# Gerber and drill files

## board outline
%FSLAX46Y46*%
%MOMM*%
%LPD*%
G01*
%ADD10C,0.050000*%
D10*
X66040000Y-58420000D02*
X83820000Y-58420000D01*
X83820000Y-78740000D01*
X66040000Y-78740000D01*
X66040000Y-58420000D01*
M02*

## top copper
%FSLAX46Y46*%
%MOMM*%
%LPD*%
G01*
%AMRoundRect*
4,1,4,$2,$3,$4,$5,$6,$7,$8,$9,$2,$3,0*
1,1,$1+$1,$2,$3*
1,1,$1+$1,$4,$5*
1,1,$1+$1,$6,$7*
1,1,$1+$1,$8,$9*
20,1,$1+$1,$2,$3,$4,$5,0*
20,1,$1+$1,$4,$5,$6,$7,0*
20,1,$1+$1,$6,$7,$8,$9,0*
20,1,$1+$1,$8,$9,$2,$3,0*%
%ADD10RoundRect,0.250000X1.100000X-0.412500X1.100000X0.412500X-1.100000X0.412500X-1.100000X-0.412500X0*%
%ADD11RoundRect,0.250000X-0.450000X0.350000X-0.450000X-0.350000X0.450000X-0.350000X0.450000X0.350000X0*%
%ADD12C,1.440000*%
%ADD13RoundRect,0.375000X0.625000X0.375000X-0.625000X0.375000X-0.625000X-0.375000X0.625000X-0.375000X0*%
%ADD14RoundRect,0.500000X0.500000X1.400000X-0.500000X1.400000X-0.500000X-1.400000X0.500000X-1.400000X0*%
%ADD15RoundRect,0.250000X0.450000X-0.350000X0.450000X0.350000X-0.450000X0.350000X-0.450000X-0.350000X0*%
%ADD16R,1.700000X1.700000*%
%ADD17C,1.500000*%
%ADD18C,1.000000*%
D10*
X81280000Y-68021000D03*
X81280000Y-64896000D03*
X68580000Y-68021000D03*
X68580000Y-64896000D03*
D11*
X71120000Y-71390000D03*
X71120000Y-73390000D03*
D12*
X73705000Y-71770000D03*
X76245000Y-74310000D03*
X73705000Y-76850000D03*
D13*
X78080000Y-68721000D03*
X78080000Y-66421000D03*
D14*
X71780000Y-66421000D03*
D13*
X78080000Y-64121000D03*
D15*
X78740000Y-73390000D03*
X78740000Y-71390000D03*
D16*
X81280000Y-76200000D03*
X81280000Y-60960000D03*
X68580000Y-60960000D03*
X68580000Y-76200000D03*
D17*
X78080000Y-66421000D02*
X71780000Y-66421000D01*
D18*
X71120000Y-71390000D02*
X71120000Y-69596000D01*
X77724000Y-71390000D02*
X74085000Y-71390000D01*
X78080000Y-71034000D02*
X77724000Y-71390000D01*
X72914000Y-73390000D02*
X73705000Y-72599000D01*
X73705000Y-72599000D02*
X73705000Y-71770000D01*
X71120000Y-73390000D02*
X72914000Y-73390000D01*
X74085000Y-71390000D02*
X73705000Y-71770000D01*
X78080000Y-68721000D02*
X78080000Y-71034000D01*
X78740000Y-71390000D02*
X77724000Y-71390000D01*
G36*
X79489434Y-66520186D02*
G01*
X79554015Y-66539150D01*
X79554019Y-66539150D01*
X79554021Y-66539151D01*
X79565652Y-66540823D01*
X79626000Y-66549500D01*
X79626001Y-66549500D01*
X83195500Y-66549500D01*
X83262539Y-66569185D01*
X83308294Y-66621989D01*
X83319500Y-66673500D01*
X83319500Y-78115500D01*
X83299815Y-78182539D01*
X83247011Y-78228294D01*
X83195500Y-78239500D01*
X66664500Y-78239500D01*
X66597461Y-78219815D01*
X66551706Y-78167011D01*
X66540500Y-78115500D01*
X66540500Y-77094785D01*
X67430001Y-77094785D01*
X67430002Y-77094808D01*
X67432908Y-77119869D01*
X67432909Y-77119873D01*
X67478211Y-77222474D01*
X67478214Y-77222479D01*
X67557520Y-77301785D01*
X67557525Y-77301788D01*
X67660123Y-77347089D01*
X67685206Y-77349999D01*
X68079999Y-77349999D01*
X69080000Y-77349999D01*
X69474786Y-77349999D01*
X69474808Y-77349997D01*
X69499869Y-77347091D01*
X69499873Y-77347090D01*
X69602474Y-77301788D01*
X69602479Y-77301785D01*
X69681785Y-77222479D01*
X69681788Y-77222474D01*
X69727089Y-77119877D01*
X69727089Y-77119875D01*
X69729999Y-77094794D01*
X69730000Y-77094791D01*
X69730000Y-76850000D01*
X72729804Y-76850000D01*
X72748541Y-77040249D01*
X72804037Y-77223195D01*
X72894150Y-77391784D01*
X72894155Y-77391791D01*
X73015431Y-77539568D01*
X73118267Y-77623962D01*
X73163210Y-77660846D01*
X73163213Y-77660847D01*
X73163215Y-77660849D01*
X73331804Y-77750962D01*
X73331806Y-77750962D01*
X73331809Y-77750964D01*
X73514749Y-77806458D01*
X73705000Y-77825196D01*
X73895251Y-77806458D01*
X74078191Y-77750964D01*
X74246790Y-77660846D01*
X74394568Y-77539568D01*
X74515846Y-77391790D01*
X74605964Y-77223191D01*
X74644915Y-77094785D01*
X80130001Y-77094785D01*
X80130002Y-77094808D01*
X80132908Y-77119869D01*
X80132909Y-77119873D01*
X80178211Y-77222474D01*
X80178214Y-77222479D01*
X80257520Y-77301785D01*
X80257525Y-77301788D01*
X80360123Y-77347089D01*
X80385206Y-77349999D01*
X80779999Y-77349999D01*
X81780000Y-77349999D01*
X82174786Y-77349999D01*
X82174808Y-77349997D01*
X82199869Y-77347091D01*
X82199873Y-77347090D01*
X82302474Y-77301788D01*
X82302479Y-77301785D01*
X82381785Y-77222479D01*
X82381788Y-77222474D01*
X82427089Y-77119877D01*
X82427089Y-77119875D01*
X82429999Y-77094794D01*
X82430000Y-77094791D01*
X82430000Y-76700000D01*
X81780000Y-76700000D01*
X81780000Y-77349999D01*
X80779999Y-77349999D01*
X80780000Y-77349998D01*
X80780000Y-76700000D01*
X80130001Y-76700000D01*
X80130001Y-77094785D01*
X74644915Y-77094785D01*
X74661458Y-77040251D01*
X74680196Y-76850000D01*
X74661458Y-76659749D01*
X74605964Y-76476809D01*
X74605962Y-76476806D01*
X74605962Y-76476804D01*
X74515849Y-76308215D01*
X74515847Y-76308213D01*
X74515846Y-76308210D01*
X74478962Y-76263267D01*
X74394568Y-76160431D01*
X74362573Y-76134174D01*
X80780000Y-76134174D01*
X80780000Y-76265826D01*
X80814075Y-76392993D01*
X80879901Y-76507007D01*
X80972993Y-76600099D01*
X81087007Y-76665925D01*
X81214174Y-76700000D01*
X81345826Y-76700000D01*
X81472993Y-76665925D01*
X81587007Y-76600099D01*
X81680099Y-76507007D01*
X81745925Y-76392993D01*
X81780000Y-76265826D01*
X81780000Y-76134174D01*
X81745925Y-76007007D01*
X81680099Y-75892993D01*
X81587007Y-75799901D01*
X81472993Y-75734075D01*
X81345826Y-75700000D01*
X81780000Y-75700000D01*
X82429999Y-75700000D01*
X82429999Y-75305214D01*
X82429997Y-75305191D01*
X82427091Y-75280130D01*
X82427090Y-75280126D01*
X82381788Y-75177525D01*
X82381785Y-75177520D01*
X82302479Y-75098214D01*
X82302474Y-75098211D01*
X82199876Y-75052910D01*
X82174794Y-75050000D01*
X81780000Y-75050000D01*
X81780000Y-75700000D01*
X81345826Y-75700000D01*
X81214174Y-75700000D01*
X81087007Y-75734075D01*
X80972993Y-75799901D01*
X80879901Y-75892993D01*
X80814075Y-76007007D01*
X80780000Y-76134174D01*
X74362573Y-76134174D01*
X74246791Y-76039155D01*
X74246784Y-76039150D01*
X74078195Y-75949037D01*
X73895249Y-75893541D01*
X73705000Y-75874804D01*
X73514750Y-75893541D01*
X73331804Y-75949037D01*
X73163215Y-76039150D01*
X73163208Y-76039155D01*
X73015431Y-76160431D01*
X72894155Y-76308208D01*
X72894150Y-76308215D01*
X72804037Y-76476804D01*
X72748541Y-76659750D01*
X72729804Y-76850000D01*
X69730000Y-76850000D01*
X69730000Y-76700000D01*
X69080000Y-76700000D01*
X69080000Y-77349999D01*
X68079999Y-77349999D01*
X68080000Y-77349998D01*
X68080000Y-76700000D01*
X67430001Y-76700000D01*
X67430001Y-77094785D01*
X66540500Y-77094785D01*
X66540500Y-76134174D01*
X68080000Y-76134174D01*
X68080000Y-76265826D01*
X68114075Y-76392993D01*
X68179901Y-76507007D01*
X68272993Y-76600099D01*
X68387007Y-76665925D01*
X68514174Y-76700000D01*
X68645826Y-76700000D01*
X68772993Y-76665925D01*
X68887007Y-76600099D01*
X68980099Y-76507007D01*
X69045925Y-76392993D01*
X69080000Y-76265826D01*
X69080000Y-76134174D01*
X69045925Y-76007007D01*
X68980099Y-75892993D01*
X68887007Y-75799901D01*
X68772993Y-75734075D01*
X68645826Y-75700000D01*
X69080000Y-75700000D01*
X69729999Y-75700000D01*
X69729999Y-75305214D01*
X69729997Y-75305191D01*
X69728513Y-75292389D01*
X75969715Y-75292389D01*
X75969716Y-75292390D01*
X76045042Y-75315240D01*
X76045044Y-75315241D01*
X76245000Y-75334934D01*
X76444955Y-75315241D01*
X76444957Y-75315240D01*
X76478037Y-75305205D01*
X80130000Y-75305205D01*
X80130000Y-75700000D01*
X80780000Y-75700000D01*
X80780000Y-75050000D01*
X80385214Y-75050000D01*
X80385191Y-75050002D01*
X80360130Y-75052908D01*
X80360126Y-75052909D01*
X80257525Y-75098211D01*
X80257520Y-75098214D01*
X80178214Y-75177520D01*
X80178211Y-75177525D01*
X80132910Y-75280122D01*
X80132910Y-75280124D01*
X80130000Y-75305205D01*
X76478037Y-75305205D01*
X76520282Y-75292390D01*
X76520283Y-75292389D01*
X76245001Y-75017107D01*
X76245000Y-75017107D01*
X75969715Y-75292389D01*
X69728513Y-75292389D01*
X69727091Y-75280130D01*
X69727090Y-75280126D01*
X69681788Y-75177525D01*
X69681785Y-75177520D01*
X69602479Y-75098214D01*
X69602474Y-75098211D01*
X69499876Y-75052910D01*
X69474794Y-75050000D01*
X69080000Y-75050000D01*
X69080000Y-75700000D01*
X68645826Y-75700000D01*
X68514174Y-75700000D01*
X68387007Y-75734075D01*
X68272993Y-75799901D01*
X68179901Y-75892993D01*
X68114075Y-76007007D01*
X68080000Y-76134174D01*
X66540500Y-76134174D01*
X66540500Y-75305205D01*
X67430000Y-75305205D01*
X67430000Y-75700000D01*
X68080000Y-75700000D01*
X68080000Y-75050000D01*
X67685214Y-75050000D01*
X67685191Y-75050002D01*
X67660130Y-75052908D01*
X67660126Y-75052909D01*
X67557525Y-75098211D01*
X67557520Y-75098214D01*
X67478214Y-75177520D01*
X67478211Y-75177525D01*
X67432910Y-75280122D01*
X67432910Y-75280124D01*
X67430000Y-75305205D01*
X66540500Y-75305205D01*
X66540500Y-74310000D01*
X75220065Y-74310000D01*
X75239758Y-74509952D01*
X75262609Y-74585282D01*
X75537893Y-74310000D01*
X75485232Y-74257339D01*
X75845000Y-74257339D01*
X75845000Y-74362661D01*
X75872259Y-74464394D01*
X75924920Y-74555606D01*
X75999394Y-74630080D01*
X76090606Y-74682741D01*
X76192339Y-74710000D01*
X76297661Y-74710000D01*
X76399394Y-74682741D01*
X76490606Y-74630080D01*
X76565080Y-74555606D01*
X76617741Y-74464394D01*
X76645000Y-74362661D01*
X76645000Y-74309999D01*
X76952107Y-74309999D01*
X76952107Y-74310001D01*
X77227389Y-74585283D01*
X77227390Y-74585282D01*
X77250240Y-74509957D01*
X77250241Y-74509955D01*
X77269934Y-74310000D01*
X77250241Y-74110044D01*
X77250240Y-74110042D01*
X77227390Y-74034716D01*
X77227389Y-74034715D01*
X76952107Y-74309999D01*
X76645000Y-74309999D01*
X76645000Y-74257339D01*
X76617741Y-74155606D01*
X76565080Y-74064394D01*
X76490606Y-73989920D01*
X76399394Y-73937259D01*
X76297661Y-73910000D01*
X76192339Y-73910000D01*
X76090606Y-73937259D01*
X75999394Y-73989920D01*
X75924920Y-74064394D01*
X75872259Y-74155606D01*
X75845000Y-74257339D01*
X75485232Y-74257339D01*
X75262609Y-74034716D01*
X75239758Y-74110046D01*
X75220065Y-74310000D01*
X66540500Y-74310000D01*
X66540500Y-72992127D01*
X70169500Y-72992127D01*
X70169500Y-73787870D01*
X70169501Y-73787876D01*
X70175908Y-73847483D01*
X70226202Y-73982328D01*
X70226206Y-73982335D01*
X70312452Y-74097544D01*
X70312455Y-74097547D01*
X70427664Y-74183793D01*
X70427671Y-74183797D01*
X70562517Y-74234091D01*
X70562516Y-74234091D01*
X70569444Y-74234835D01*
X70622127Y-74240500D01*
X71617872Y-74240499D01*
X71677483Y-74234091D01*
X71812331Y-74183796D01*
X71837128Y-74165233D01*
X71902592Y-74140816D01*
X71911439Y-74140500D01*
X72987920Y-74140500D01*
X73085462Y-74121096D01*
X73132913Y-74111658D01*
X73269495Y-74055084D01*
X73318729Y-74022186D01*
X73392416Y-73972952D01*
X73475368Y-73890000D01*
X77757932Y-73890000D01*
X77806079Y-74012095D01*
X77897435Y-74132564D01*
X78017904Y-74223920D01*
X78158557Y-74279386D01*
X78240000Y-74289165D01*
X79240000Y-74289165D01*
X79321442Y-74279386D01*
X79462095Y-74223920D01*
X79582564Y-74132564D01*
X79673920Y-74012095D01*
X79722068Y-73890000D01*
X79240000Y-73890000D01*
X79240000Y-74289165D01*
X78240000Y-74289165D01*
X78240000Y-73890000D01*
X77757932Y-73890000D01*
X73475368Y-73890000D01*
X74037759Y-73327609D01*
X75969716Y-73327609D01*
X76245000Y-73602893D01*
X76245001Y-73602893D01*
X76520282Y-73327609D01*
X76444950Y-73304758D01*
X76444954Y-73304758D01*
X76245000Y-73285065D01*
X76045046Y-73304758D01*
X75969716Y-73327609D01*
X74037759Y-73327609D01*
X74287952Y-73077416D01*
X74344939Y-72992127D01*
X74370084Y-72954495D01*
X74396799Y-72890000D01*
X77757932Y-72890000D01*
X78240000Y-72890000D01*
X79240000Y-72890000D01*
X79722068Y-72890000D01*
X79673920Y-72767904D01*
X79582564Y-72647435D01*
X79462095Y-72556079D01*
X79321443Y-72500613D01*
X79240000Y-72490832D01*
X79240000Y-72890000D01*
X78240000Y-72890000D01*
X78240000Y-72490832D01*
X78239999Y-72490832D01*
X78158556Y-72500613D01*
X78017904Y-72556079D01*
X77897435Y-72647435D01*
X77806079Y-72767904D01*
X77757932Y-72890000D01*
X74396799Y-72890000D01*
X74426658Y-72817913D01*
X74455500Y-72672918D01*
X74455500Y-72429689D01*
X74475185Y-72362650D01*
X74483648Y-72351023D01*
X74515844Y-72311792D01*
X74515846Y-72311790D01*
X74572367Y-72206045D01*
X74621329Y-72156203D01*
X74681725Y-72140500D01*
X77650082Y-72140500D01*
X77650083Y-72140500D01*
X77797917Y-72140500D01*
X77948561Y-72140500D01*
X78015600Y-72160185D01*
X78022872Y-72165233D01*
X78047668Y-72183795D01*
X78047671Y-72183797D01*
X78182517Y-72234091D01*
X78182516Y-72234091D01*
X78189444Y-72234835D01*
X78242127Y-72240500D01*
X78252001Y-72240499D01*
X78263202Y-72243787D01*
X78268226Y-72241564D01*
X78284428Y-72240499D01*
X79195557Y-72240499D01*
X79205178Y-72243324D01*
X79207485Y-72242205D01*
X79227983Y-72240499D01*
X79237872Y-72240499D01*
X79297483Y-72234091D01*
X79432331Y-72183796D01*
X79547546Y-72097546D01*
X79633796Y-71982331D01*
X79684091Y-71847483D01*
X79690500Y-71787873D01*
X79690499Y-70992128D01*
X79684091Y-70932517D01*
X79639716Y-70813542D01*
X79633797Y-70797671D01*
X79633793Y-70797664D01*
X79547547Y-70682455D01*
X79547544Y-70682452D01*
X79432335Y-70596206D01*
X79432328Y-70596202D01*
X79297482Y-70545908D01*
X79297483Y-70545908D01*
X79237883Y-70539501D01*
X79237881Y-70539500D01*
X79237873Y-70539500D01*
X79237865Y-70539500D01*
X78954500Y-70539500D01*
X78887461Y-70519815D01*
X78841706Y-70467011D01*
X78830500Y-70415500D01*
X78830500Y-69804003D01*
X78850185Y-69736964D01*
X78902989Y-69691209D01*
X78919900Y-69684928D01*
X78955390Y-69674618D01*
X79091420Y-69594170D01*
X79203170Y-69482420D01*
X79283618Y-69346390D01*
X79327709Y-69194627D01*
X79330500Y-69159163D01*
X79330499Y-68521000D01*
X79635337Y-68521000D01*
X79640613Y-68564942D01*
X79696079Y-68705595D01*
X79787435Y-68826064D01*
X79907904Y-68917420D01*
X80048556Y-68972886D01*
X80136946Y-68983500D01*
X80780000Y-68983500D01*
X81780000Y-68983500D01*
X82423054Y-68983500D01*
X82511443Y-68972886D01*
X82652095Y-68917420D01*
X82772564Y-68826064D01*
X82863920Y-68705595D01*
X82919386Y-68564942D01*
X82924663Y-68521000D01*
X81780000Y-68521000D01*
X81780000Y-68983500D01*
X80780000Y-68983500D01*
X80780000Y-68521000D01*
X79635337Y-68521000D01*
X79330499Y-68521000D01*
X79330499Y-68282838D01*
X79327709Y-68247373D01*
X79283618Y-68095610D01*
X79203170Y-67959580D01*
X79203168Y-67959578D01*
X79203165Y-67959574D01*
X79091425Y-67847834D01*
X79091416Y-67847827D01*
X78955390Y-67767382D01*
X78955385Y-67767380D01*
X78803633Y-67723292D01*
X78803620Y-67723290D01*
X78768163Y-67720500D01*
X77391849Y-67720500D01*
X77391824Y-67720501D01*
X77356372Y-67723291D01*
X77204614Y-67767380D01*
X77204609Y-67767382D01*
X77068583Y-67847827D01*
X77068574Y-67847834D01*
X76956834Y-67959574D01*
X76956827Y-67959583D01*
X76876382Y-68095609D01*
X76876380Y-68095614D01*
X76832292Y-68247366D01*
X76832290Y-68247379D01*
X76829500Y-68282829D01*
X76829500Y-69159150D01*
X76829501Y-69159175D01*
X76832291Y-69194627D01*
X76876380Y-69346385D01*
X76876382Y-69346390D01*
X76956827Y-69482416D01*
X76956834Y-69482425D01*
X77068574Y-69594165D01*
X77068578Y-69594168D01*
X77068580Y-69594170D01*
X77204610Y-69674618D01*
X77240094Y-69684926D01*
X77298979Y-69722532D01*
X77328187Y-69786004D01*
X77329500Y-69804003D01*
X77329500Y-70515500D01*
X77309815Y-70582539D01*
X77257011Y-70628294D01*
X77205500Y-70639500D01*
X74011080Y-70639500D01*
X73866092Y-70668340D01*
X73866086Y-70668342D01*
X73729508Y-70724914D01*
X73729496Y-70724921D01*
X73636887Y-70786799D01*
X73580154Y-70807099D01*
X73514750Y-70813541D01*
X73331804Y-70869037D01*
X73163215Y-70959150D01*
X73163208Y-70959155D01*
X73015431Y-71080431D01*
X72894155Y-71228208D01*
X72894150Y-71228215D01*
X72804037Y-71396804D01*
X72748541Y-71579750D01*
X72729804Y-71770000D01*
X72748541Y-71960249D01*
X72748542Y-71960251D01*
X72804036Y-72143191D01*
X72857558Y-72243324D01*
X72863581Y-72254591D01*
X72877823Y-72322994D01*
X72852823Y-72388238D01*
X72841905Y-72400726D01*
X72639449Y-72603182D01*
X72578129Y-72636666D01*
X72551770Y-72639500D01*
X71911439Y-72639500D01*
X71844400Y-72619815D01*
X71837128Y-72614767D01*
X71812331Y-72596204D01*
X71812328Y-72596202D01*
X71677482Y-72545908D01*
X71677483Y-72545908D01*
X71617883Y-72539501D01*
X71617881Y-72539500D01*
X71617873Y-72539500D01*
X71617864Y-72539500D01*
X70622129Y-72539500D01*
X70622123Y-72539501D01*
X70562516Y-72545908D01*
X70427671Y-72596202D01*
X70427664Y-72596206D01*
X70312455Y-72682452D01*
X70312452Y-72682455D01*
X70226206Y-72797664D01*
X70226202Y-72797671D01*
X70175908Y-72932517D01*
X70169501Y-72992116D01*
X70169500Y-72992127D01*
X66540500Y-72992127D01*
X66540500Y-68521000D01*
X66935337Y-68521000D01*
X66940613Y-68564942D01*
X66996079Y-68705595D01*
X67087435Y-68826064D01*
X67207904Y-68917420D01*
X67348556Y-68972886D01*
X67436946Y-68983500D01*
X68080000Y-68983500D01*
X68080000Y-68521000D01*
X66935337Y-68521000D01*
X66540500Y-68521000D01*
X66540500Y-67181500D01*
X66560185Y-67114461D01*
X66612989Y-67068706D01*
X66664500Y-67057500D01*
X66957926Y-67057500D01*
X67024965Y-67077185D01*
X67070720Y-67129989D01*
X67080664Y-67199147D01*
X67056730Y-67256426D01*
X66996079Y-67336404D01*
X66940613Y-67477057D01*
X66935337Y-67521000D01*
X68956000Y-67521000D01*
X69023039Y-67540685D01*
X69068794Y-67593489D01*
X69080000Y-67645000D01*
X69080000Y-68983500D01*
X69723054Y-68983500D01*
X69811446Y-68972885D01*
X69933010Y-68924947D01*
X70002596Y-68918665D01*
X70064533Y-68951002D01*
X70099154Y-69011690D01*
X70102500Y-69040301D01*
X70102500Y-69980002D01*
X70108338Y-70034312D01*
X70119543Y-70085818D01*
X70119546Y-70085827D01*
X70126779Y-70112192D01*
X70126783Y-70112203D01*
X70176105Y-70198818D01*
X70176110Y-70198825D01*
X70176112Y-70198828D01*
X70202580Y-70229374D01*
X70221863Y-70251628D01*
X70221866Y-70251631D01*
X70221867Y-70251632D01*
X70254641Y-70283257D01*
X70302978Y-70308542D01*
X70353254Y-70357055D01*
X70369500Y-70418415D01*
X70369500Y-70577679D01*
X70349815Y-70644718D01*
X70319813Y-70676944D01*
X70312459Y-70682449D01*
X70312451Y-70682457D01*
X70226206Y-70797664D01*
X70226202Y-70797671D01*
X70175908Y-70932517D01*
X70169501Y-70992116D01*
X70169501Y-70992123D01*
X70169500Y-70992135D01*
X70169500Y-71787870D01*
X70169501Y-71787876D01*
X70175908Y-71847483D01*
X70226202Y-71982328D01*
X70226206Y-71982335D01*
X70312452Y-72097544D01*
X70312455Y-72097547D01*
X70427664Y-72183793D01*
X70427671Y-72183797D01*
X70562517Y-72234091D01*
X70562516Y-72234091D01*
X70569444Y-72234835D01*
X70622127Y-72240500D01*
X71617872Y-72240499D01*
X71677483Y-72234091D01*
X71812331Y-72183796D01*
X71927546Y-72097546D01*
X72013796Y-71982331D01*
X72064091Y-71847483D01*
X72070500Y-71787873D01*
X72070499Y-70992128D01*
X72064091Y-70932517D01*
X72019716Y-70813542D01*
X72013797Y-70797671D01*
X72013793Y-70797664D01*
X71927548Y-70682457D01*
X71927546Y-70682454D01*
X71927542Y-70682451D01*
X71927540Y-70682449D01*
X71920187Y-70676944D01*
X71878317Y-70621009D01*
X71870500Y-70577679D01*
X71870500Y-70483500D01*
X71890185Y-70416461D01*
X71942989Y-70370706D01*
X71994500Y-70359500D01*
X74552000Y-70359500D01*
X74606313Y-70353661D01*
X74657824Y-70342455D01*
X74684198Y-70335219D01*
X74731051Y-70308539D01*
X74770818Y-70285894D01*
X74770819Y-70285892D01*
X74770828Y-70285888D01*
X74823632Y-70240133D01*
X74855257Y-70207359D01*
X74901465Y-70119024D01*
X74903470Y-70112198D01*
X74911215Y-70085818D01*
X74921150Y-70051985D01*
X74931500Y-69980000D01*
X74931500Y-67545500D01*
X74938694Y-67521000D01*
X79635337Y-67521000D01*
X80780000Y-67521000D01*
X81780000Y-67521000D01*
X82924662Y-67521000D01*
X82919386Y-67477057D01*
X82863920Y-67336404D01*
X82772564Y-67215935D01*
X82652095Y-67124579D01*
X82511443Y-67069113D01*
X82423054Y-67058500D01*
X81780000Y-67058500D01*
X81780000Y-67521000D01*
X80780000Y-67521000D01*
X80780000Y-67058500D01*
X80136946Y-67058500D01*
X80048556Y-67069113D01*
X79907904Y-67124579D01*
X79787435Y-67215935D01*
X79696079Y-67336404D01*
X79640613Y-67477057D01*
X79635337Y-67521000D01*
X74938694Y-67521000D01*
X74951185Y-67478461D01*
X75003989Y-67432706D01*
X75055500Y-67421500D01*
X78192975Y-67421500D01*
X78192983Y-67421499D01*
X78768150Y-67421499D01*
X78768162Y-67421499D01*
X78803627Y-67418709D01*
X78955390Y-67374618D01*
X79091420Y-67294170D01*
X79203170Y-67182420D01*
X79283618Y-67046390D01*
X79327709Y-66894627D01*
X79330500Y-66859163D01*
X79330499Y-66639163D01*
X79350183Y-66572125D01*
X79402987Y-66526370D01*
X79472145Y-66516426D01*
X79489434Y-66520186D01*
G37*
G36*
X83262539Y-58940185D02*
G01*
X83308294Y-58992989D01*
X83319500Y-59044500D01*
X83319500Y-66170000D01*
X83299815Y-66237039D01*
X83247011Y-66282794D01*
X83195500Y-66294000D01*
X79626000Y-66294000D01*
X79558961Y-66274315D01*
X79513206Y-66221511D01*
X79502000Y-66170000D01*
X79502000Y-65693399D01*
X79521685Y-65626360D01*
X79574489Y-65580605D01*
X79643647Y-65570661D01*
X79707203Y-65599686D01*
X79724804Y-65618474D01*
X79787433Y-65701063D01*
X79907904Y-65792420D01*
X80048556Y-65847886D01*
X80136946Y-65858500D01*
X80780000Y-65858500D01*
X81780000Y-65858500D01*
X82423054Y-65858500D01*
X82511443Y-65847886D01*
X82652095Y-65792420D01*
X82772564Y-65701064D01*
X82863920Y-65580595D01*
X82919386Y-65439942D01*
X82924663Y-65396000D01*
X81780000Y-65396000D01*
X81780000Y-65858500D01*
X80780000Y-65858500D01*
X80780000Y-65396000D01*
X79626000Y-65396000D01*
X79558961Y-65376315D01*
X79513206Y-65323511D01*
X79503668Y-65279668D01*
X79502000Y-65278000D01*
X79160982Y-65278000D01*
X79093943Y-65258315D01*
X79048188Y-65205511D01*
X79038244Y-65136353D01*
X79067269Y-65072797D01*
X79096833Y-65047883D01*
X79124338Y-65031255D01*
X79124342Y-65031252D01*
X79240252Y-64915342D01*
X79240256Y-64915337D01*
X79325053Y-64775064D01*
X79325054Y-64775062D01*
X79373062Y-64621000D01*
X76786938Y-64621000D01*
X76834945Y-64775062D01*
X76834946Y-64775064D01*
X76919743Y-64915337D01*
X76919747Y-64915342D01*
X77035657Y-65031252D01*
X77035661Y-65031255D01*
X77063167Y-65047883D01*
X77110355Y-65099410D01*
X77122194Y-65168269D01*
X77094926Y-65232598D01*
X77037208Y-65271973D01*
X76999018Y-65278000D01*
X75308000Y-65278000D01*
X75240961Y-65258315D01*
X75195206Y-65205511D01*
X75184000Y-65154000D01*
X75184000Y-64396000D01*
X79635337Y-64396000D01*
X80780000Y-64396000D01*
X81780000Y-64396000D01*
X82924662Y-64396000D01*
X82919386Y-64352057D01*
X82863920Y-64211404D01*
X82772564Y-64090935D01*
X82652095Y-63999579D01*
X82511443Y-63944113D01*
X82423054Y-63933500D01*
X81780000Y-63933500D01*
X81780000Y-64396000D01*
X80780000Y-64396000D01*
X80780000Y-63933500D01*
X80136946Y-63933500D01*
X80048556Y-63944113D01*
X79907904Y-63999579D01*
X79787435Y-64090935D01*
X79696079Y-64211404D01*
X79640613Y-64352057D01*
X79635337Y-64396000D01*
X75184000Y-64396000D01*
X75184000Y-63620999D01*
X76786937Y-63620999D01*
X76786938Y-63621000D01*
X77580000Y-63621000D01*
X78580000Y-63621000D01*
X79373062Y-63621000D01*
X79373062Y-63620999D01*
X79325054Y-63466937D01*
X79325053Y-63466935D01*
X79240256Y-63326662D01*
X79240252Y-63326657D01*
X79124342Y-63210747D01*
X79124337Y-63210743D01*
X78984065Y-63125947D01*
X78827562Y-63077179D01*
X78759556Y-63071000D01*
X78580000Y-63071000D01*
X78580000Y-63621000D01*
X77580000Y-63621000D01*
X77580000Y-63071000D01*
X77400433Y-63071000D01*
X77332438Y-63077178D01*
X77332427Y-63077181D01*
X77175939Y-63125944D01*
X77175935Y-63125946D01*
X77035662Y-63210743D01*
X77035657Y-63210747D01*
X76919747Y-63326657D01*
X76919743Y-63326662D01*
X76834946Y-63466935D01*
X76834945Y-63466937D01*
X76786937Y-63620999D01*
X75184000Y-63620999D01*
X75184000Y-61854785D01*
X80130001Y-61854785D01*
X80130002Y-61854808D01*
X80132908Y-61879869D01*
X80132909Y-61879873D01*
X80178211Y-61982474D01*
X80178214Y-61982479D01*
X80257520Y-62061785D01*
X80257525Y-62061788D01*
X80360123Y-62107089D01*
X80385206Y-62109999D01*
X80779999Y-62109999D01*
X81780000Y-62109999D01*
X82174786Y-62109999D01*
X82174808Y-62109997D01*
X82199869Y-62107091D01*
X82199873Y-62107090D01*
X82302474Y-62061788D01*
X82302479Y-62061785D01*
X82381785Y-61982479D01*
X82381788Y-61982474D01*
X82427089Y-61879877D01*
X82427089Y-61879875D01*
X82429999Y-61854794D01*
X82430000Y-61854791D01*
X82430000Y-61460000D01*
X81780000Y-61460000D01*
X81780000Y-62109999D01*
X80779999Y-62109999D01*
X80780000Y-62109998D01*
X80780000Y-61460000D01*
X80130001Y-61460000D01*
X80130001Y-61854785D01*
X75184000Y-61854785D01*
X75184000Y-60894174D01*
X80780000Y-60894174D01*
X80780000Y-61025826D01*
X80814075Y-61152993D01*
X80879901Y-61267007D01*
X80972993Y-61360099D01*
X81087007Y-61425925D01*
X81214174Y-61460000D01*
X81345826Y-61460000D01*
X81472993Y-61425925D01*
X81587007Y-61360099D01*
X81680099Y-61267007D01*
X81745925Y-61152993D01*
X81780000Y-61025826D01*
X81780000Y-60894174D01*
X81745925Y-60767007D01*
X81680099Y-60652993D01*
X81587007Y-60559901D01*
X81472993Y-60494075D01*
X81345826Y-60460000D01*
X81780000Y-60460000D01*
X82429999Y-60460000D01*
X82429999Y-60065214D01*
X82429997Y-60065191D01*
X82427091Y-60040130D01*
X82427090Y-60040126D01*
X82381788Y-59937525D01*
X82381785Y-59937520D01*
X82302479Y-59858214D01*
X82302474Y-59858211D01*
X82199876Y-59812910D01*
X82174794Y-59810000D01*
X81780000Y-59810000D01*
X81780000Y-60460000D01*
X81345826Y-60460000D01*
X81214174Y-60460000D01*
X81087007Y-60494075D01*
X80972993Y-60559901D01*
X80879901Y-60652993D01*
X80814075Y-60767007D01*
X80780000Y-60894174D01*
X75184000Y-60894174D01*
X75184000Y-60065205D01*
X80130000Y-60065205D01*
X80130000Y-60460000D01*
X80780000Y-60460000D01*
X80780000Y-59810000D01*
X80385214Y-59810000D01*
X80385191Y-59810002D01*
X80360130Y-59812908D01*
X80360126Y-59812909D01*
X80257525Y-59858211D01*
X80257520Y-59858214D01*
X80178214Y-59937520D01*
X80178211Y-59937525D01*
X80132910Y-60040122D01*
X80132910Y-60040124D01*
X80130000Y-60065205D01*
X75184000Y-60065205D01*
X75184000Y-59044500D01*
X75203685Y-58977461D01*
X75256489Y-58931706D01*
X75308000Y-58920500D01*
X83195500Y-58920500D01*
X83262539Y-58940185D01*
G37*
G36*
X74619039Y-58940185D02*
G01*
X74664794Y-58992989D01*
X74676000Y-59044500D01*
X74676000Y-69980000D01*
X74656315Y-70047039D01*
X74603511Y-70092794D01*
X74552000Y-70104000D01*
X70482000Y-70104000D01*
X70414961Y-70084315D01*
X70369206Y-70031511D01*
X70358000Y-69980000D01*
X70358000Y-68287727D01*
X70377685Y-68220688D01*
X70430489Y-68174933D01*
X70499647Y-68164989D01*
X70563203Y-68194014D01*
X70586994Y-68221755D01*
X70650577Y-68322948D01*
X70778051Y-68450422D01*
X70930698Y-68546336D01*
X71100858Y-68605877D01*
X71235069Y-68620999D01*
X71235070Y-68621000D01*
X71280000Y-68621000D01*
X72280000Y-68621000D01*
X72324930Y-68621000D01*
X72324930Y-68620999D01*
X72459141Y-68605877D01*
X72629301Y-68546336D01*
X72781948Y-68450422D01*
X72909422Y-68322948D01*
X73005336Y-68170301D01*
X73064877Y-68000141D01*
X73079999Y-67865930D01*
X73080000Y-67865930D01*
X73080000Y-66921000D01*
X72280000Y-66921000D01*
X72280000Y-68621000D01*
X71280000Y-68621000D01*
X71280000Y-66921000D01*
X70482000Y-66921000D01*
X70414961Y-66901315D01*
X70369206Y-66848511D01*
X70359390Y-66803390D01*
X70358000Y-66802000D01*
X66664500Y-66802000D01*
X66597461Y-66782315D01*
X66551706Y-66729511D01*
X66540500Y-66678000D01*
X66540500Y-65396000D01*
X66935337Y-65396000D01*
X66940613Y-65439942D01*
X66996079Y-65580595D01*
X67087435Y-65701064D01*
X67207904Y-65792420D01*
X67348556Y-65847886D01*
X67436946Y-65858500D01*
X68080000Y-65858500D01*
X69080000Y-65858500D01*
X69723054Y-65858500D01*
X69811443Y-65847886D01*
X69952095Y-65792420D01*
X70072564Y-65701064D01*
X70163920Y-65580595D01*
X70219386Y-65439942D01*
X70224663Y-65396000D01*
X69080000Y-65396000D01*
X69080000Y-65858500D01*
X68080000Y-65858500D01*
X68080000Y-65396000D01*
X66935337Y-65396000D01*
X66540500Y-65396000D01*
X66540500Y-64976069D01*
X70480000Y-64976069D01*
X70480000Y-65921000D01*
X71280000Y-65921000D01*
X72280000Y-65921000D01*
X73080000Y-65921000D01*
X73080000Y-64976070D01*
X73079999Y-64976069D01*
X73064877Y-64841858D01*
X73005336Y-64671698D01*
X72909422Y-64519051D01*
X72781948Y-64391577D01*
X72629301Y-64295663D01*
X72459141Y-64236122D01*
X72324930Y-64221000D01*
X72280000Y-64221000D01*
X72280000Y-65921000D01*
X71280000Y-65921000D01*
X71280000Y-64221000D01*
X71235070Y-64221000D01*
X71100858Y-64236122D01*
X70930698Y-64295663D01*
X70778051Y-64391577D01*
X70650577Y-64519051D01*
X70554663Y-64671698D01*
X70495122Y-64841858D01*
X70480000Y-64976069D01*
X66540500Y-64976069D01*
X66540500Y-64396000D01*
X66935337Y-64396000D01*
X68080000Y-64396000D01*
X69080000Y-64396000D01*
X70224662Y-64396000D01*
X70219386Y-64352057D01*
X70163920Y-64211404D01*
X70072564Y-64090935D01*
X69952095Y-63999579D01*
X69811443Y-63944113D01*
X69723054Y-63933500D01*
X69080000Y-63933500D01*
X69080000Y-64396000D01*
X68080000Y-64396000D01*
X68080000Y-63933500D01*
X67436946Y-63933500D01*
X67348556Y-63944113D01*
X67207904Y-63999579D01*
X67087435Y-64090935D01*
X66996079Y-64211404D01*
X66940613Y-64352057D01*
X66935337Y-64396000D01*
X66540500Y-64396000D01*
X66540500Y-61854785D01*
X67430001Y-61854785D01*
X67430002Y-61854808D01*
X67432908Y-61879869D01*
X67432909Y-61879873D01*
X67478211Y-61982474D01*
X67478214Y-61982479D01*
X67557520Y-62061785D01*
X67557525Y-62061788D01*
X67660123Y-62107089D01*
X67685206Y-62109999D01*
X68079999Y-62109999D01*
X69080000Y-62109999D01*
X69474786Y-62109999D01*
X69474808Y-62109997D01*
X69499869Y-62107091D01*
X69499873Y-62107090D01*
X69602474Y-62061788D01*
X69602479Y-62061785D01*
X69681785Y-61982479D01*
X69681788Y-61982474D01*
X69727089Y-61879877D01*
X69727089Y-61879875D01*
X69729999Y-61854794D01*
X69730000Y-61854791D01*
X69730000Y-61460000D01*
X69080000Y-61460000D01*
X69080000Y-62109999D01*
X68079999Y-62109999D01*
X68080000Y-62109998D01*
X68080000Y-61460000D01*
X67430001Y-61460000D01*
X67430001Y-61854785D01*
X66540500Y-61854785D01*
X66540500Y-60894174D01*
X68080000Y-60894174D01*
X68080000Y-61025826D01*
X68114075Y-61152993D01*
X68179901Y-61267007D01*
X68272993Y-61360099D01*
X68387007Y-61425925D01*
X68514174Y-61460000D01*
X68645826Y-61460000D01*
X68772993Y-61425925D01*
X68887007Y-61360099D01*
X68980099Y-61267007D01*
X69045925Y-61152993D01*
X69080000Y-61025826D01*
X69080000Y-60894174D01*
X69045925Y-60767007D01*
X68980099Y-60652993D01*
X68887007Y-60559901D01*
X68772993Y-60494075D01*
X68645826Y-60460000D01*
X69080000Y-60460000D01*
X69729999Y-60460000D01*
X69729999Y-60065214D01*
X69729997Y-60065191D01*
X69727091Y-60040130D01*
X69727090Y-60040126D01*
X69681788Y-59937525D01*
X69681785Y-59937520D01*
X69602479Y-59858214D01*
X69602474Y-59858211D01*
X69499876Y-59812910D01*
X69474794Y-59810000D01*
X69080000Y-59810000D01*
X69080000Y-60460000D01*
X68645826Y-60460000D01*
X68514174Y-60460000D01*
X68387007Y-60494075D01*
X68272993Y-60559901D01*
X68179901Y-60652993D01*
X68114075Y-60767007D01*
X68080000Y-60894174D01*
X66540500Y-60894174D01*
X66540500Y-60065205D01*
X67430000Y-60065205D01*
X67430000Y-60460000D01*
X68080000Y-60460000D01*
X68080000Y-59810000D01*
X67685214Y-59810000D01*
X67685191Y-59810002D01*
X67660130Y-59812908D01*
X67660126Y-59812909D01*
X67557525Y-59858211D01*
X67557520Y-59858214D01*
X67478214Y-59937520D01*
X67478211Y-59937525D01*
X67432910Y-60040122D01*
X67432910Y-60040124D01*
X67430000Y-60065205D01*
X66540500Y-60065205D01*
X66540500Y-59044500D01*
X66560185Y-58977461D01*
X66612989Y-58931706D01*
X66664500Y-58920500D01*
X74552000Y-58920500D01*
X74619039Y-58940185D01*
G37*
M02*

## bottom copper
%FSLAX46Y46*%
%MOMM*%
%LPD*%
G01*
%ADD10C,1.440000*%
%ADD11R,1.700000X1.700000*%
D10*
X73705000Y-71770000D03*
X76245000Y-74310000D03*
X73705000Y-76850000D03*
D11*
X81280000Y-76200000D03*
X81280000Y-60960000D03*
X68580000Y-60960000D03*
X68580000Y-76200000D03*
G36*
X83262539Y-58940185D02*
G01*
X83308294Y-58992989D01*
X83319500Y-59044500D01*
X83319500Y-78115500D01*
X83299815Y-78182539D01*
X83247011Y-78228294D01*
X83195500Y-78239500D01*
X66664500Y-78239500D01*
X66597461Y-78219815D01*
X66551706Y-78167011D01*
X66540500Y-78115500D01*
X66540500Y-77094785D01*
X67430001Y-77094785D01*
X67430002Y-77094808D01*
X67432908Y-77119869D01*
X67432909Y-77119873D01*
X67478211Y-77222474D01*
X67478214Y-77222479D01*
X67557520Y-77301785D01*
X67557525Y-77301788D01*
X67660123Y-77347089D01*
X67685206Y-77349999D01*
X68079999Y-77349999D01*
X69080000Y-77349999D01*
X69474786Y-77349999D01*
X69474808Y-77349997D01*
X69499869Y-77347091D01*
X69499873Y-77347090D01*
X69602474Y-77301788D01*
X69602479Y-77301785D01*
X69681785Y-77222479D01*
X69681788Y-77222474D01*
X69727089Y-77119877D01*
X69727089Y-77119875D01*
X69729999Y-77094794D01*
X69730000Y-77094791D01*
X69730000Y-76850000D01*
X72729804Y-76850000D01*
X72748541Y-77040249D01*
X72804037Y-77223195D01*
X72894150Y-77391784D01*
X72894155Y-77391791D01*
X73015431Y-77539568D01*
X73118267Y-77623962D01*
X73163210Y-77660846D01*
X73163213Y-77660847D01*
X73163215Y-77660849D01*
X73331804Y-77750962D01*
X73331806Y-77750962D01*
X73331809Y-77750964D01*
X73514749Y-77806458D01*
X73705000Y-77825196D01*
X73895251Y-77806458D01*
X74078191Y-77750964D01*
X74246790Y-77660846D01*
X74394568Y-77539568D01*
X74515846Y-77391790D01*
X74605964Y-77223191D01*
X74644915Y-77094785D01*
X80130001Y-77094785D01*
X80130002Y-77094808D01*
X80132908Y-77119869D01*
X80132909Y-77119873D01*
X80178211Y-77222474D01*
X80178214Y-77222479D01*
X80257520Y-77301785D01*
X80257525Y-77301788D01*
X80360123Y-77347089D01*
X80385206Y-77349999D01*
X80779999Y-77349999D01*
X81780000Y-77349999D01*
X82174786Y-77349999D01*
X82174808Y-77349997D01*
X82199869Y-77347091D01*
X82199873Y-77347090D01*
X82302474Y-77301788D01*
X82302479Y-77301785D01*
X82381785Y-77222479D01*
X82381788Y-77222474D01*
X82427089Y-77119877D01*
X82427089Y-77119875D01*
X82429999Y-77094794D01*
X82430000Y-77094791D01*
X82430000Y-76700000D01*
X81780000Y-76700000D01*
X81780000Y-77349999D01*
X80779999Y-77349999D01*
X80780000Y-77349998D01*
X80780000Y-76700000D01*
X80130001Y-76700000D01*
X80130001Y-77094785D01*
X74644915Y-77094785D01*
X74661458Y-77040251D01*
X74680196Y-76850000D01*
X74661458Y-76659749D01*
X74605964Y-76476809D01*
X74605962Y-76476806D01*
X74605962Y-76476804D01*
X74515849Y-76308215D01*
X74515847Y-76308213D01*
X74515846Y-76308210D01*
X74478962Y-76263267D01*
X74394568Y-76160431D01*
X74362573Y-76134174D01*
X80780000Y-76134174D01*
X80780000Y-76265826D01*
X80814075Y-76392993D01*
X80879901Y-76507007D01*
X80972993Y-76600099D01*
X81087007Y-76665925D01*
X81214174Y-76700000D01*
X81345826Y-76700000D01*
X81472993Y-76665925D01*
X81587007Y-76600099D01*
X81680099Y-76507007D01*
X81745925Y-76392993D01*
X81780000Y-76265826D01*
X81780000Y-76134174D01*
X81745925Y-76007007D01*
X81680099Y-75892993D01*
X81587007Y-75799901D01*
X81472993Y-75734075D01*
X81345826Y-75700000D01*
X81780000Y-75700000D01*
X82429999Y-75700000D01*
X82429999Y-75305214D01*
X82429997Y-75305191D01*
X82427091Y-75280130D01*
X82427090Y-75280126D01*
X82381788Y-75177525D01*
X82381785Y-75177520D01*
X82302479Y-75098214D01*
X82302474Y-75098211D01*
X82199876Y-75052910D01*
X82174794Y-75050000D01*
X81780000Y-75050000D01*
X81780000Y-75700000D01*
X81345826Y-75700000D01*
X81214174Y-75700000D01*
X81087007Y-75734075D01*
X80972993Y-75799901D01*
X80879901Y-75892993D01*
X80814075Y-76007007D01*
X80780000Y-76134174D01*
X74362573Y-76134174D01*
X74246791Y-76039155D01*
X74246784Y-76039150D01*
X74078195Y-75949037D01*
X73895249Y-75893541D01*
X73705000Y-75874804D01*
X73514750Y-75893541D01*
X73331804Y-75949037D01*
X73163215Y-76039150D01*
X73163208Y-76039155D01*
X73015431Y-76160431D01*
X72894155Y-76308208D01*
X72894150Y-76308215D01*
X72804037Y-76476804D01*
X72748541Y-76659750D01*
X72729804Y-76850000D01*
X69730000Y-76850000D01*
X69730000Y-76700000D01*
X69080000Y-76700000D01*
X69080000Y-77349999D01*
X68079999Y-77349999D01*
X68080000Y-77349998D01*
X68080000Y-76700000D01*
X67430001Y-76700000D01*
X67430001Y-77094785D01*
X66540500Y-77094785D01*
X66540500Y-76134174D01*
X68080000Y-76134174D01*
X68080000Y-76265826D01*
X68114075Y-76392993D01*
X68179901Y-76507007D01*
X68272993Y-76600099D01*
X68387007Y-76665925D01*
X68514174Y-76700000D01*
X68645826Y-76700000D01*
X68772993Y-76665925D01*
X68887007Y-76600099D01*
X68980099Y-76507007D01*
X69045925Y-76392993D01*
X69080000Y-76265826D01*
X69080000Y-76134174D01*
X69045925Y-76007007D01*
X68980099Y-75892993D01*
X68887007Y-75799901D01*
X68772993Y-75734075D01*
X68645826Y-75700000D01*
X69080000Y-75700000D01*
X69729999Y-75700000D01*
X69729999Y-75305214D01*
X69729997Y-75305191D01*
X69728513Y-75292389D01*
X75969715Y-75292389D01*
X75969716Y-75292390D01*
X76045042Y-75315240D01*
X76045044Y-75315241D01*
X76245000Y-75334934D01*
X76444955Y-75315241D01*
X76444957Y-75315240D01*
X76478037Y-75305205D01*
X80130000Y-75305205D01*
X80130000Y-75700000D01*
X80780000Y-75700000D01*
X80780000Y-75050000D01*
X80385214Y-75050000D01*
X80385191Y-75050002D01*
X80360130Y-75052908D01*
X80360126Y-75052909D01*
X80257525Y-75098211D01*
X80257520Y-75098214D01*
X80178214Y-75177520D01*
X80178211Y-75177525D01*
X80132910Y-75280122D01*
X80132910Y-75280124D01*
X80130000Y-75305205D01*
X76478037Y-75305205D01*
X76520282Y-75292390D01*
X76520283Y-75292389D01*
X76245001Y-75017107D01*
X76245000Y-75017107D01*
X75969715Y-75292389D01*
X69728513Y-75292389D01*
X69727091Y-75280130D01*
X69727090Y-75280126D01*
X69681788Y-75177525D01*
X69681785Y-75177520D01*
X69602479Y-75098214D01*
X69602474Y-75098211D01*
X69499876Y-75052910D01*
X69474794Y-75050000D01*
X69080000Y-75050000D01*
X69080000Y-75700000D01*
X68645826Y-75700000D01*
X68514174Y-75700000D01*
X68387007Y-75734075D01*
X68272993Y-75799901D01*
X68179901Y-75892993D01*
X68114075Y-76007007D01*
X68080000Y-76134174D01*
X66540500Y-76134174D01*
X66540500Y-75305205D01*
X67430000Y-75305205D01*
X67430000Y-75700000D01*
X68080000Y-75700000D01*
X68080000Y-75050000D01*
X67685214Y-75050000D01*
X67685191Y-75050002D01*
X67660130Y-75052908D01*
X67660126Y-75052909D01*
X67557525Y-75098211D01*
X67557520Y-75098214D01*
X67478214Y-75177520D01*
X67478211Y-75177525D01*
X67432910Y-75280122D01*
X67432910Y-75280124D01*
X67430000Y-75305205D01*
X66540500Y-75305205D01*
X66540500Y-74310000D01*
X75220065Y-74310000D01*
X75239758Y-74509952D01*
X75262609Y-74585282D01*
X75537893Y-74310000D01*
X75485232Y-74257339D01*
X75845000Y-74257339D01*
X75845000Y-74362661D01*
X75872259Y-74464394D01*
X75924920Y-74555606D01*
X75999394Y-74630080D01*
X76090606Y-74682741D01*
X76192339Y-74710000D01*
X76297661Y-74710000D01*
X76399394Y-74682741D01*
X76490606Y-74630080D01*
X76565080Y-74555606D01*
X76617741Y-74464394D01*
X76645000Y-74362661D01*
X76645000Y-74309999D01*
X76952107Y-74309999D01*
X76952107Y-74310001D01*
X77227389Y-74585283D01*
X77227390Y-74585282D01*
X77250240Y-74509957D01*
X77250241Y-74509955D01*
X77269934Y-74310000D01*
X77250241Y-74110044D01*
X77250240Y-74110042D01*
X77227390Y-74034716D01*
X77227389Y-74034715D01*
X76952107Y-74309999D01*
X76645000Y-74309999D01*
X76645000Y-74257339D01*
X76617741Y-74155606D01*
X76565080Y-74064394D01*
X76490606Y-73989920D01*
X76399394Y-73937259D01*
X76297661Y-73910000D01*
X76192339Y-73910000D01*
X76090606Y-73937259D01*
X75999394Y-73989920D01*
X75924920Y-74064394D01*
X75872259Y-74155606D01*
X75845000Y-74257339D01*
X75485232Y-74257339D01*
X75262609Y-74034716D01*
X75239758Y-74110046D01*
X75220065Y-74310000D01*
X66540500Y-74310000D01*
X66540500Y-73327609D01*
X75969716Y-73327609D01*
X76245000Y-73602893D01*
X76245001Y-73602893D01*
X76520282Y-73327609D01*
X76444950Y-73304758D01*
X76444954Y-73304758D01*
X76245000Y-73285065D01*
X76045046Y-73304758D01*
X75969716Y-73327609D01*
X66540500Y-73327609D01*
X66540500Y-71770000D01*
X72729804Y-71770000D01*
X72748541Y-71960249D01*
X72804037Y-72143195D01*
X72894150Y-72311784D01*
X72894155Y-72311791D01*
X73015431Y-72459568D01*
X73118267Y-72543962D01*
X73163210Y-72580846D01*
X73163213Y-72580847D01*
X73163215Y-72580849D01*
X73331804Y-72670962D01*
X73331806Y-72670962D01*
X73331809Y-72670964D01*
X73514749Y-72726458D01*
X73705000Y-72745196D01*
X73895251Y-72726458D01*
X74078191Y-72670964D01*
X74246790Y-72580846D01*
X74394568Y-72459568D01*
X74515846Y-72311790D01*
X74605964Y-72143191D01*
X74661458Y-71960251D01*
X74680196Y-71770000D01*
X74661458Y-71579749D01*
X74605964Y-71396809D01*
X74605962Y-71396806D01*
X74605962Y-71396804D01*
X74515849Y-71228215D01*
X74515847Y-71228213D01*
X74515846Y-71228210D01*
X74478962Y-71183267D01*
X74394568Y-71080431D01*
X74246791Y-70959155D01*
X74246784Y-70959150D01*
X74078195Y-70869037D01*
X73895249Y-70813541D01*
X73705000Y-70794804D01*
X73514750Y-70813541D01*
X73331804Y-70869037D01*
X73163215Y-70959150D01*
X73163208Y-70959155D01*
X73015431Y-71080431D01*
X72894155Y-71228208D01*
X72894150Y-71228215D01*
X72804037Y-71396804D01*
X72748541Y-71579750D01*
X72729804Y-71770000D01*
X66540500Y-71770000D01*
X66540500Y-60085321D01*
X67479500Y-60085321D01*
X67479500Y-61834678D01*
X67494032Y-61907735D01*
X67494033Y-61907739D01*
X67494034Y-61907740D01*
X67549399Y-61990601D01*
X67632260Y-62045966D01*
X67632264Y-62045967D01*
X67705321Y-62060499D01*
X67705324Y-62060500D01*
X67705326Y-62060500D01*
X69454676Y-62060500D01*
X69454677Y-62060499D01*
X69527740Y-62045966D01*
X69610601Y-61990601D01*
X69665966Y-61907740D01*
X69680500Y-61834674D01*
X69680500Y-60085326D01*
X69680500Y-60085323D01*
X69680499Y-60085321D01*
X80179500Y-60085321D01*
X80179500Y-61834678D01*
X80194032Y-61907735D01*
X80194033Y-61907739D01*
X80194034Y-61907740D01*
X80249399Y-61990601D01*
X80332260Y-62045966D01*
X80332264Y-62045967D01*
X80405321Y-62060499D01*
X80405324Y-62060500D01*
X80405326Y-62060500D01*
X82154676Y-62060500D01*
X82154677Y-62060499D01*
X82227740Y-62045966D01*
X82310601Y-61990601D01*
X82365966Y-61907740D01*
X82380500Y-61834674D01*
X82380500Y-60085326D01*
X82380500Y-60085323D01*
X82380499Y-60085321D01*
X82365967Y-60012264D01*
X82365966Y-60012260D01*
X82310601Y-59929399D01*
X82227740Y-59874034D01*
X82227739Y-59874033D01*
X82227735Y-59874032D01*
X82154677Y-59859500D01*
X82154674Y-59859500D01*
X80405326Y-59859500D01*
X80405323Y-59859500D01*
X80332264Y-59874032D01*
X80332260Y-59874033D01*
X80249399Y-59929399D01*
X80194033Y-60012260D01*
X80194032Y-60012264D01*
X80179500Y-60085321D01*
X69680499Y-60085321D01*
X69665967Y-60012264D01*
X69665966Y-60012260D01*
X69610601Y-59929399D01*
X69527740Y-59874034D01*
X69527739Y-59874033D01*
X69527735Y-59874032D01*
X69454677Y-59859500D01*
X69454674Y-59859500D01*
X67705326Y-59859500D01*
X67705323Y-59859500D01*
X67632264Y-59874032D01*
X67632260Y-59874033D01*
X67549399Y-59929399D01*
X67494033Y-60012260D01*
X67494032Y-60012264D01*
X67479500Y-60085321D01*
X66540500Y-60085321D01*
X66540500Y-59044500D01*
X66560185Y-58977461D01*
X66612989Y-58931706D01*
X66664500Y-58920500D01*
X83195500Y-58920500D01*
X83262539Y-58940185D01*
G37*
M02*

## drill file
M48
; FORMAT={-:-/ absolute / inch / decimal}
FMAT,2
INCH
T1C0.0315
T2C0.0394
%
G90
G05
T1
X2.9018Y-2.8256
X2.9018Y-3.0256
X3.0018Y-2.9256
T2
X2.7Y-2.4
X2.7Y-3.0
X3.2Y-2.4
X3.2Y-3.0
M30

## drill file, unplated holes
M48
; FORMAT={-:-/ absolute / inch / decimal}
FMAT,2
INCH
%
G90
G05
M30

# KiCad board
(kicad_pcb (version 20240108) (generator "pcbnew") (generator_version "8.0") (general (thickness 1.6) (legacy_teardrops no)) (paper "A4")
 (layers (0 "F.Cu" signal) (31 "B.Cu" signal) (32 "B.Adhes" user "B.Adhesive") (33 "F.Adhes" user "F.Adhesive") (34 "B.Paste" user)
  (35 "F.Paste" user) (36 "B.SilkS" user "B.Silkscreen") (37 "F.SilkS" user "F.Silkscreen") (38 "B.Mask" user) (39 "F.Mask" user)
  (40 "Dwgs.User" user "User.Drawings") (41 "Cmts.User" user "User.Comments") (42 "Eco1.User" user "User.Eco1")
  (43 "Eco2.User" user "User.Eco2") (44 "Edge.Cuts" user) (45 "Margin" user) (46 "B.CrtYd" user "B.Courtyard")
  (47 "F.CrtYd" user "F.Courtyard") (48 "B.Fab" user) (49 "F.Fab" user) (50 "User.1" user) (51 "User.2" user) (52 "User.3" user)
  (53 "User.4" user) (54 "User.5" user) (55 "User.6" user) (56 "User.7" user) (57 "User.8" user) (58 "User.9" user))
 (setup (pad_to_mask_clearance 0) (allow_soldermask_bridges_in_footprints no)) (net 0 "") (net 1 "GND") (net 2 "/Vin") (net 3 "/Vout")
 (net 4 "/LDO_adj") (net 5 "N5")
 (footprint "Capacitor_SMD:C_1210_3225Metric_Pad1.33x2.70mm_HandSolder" (layer "F.Cu") (at 81.28 66.4585 90)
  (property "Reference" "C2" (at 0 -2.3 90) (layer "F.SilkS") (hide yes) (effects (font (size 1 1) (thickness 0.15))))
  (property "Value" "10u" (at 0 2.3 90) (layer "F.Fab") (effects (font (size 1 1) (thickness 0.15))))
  (pad "1" smd roundrect (at -1.5625 0 90) (size 1.325 2.7) (layers "F.Cu" "F.Paste" "F.Mask") (roundrect_rratio 0.188679) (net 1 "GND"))
  (pad "2" smd roundrect (at 1.5625 0 90) (size 1.325 2.7) (layers "F.Cu" "F.Paste" "F.Mask") (roundrect_rratio 0.188679) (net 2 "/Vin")))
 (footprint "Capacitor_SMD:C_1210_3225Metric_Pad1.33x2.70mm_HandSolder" (layer "F.Cu") (at 68.58 66.4585 90)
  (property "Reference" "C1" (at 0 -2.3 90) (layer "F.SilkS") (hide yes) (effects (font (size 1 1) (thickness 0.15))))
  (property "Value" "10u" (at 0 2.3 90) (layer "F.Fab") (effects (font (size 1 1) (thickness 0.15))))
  (pad "1" smd roundrect (at -1.5625 0 90) (size 1.325 2.7) (layers "F.Cu" "F.Paste" "F.Mask") (roundrect_rratio 0.188679) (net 1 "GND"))
  (pad "2" smd roundrect (at 1.5625 0 90) (size 1.325 2.7) (layers "F.Cu" "F.Paste" "F.Mask") (roundrect_rratio 0.188679) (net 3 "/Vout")))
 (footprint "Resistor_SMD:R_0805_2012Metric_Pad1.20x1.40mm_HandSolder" (layer "F.Cu") (at 71.12 72.39 -90)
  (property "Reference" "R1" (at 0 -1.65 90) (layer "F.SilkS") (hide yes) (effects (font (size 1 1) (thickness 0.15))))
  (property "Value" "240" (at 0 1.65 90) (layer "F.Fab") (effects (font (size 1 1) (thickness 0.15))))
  (pad "1" smd roundrect (at -1 0 270) (size 1.2 1.4) (layers "F.Cu" "F.Paste" "F.Mask") (roundrect_rratio 0.208333) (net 3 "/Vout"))
  (pad "2" smd roundrect (at 1 0 270) (size 1.2 1.4) (layers "F.Cu" "F.Paste" "F.Mask") (roundrect_rratio 0.208333) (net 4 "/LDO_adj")))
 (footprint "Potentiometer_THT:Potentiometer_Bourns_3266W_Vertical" (layer "F.Cu") (at 73.705 71.77 90)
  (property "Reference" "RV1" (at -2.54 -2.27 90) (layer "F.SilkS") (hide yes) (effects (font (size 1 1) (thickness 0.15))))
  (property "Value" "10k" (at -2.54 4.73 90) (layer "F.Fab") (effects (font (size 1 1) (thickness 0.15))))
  (pad "1" thru_hole circle (at 0 0 90) (size 1.44 1.44) (drill 0.8) (layers "*.Cu" "*.Mask") (remove_unused_layers no) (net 4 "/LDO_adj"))
  (pad "2" thru_hole circle (at -2.54 2.54 90) (size 1.44 1.44) (drill 0.8) (layers "*.Cu" "*.Mask") (remove_unused_layers no) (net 1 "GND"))
  (pad "3" thru_hole circle (at -5.08 0 90) (size 1.44 1.44) (drill 0.8) (layers "*.Cu" "*.Mask") (remove_unused_layers no) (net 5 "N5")))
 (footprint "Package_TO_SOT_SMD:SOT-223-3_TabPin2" (layer "F.Cu") (at 74.93 66.421 180)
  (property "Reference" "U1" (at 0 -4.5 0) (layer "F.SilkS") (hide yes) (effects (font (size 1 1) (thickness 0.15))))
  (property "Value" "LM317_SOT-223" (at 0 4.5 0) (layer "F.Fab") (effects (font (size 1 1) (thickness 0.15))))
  (pad "1" smd roundrect (at -3.15 -2.3 180) (size 2 1.5) (layers "F.Cu" "F.Paste" "F.Mask") (roundrect_rratio 0.25) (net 4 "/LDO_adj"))
  (pad "2" smd roundrect (at -3.15 0 180) (size 2 1.5) (layers "F.Cu" "F.Paste" "F.Mask") (roundrect_rratio 0.25) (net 3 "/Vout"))
  (pad "2" smd roundrect (at 3.15 0 180) (size 2 3.8) (layers "F.Cu" "F.Paste" "F.Mask") (roundrect_rratio 0.25) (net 3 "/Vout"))
  (pad "3" smd roundrect (at -3.15 2.3 180) (size 2 1.5) (layers "F.Cu" "F.Paste" "F.Mask") (roundrect_rratio 0.25) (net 2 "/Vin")))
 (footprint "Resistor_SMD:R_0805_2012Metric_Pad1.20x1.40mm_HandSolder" (layer "F.Cu") (at 78.74 72.39 90)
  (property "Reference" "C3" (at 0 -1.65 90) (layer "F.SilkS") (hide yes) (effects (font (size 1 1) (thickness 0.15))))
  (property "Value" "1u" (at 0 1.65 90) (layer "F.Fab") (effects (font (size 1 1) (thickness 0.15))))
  (pad "1" smd roundrect (at -1 0 90) (size 1.2 1.4) (layers "F.Cu" "F.Paste" "F.Mask") (roundrect_rratio 0.208333) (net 1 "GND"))
  (pad "2" smd roundrect (at 1 0 90) (size 1.2 1.4) (layers "F.Cu" "F.Paste" "F.Mask") (roundrect_rratio 0.208333) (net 4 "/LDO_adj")))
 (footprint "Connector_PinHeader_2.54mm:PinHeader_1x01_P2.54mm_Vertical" (layer "B.Cu") (at 81.28 76.2 180)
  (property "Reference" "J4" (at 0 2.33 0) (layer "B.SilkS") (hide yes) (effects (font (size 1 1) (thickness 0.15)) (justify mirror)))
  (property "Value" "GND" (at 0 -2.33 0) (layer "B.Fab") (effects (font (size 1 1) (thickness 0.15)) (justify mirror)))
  (pad "1" thru_hole rect (at 0 0 180) (size 1.7 1.7) (drill 1) (layers "*.Cu" "*.Mask") (remove_unused_layers no) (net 1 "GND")))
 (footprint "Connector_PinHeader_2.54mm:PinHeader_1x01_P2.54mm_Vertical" (layer "B.Cu") (at 81.28 60.96 180)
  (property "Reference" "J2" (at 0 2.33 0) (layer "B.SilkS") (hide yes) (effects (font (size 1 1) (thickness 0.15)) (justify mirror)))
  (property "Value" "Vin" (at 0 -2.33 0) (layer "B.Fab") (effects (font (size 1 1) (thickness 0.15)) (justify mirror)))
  (pad "1" thru_hole rect (at 0 0 180) (size 1.7 1.7) (drill 1) (layers "*.Cu" "*.Mask") (remove_unused_layers no) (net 2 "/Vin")))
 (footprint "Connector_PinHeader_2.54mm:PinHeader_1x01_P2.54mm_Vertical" (layer "B.Cu") (at 68.58 60.96 180)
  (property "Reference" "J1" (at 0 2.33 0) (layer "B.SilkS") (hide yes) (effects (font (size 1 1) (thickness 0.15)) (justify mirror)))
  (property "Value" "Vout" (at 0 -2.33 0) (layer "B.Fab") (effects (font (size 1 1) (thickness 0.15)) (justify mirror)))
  (pad "1" thru_hole rect (at 0 0 180) (size 1.7 1.7) (drill 1) (layers "*.Cu" "*.Mask") (remove_unused_layers no) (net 3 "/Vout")))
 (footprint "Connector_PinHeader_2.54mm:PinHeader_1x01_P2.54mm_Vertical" (layer "B.Cu") (at 68.58 76.2 180)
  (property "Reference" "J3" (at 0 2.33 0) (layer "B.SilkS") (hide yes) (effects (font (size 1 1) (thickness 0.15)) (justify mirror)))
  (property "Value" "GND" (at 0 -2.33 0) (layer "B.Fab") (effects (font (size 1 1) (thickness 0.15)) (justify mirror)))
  (pad "1" thru_hole rect (at 0 0 180) (size 1.7 1.7) (drill 1) (layers "*.Cu" "*.Mask") (remove_unused_layers no) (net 1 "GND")))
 (gr_rect (start 66.04 58.42) (end 83.82 78.74) (stroke (width 0.05) (type default)) (fill none) (layer "Edge.Cuts"))
 (segment (start 78.08 66.421) (end 71.78 66.421) (width 1.5) (layer "F.Cu") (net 3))
 (segment (start 71.12 71.39) (end 71.12 69.596) (width 1) (layer "F.Cu") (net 3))
 (segment (start 77.724 71.39) (end 74.085 71.39) (width 1) (layer "F.Cu") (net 4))
 (segment (start 78.08 71.034) (end 77.724 71.39) (width 1) (layer "F.Cu") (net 4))
 (segment (start 72.914 73.39) (end 73.705 72.599) (width 1) (layer "F.Cu") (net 4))
 (segment (start 73.705 72.599) (end 73.705 71.77) (width 1) (layer "F.Cu") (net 4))
 (segment (start 71.12 73.39) (end 72.914 73.39) (width 1) (layer "F.Cu") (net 4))
 (segment (start 74.085 71.39) (end 73.705 71.77) (width 1) (layer "F.Cu") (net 4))
 (segment (start 78.08 68.721) (end 78.08 71.034) (width 1) (layer "F.Cu") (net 4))
 (segment (start 78.74 71.39) (end 77.724 71.39) (width 1) (layer "F.Cu") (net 4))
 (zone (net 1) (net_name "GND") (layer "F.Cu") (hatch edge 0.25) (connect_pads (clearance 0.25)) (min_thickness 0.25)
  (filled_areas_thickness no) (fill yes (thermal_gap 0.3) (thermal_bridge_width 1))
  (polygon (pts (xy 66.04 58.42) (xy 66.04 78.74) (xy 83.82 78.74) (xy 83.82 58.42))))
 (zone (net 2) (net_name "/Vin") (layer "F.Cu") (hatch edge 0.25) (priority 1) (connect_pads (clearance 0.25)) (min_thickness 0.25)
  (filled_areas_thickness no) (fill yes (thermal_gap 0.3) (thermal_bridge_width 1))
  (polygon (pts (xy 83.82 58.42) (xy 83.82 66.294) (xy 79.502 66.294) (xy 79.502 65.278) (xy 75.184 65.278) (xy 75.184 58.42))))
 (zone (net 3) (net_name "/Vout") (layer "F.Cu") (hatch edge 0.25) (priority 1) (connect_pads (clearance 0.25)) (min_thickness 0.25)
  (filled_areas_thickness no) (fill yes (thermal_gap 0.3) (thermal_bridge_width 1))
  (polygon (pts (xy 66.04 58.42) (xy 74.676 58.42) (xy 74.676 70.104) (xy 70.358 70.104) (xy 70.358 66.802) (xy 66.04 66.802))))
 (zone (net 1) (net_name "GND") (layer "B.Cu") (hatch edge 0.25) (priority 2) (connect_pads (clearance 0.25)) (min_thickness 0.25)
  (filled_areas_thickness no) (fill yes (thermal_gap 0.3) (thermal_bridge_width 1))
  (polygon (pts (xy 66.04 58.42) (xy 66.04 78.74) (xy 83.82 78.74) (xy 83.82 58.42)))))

